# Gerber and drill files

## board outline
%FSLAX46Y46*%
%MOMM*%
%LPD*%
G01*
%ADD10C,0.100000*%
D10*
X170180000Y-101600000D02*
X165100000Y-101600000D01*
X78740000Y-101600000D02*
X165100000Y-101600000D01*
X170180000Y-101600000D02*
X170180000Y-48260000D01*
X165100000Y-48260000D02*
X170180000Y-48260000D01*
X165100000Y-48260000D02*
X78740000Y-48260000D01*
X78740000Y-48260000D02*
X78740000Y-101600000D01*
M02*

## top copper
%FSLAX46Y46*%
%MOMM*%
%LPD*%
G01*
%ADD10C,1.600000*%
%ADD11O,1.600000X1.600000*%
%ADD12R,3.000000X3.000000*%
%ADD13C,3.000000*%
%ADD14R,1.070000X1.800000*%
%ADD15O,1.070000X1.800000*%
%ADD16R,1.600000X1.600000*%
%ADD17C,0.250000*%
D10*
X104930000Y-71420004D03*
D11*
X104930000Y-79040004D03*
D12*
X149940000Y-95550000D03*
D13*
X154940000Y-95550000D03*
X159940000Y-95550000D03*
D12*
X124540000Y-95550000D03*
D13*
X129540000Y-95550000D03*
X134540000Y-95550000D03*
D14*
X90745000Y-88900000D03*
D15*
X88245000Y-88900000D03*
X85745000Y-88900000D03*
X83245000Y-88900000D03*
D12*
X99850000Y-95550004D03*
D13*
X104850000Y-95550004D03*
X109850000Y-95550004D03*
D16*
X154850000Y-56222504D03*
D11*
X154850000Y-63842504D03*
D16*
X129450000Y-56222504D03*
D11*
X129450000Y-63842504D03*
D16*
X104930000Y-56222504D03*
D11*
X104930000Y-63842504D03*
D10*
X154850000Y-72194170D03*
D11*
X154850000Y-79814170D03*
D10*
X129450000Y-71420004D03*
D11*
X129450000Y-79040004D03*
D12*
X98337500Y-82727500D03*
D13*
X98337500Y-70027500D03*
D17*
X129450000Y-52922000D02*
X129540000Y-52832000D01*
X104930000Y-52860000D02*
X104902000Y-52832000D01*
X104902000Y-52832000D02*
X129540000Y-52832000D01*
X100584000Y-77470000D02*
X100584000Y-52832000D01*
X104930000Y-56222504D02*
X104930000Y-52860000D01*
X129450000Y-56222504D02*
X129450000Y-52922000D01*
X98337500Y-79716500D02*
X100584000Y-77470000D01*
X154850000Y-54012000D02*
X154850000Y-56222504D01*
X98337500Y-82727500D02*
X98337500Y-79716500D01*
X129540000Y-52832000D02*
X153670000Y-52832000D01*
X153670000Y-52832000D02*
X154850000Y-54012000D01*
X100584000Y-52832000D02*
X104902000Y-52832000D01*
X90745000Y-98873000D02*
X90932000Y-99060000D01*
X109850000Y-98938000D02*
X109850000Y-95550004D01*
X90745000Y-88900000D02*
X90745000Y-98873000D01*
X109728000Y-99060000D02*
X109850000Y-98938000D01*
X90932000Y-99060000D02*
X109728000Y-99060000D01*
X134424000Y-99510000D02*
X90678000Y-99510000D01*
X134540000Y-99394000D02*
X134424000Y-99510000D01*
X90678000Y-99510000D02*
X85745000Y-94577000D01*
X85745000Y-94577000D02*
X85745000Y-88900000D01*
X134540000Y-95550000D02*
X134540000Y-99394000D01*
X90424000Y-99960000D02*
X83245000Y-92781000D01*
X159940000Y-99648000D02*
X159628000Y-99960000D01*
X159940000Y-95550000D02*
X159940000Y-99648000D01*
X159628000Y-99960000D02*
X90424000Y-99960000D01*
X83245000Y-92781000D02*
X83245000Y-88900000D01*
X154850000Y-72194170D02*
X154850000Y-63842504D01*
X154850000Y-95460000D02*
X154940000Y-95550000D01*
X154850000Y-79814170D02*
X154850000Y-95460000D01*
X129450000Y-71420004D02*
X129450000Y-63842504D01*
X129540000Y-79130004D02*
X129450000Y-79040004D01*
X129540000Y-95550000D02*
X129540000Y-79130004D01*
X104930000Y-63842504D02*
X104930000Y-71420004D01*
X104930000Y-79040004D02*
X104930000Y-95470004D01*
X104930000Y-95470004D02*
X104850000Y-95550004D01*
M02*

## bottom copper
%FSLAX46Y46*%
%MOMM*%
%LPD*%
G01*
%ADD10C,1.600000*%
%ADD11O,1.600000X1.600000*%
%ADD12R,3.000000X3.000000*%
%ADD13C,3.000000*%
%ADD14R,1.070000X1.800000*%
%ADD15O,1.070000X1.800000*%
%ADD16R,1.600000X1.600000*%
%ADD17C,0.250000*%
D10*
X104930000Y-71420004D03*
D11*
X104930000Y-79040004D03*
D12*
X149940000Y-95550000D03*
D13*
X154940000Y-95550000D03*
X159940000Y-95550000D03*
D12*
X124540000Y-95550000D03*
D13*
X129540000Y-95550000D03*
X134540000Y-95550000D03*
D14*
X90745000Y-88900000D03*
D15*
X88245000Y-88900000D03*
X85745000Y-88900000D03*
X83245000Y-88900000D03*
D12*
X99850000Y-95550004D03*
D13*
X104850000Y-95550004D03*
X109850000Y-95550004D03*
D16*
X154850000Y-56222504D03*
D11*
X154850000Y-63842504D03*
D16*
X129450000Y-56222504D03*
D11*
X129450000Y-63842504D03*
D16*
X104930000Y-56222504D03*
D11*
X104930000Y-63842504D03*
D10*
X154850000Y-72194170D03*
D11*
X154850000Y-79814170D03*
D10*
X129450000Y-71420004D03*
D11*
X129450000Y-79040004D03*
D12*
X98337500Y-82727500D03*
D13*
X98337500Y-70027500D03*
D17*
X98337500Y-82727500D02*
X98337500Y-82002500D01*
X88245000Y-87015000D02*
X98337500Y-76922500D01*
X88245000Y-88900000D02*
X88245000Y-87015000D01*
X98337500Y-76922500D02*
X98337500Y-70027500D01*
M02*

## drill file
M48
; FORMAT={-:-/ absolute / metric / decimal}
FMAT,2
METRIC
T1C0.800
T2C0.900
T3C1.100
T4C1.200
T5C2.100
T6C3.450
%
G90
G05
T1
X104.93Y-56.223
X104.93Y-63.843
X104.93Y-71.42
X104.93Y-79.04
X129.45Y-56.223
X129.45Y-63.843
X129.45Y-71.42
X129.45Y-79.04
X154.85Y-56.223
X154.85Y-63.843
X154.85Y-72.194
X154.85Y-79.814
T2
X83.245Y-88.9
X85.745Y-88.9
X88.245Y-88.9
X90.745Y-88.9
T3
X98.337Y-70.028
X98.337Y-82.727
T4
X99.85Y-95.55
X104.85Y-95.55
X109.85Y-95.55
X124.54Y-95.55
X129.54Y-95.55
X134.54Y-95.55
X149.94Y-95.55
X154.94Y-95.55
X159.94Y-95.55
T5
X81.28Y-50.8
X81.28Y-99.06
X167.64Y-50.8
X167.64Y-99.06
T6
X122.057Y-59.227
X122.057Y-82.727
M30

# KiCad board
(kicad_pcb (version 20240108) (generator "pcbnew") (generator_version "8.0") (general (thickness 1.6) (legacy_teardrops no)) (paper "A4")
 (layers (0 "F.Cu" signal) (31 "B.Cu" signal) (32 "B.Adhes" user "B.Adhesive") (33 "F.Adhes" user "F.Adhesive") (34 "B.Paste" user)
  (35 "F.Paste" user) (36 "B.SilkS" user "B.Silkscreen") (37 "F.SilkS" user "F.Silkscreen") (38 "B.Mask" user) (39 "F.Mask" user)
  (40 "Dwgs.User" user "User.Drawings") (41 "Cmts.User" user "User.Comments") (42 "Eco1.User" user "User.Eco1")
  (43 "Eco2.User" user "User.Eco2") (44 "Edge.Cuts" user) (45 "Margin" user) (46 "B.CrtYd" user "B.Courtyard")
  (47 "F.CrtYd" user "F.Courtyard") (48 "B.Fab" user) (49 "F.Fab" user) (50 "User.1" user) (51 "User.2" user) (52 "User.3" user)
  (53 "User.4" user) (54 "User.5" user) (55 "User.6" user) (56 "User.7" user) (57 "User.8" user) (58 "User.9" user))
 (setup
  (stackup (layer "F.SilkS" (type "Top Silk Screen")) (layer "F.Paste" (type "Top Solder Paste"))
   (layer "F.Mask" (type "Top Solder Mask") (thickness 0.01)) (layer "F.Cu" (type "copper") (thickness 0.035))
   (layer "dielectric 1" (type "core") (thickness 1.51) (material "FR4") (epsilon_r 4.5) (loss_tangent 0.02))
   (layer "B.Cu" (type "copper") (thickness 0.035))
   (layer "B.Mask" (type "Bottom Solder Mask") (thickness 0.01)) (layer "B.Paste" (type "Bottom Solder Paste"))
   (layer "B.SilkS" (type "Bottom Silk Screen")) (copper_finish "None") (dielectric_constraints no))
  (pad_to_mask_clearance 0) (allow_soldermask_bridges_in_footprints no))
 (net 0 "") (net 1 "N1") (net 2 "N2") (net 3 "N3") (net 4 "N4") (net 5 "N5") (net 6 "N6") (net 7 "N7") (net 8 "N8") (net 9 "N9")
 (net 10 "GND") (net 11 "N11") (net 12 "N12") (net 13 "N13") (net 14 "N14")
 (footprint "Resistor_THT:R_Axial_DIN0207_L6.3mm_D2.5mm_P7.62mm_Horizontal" (layer "F.Cu") (at 104.93 71.420004 -90)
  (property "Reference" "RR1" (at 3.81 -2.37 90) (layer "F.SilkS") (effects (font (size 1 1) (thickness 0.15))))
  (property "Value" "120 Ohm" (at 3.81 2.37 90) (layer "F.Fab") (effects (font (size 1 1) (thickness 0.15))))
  (pad "1" thru_hole circle (at 0 0 270) (size 1.6 1.6) (drill 0.8) (layers "*.Cu" "*.Mask") (remove_unused_layers no) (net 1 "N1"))
  (pad "2" thru_hole oval (at 7.62 0 270) (size 1.6 1.6) (drill 0.8) (layers "*.Cu" "*.Mask") (remove_unused_layers no) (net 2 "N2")))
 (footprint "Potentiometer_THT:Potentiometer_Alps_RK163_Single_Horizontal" (layer "F.Cu") (at 149.94 95.55 90)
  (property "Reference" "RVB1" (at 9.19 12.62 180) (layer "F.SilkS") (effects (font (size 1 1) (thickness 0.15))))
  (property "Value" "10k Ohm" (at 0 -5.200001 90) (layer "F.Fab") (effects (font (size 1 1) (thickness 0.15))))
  (pad "1" thru_hole rect (at 0 0 270) (size 3 3) (drill 1.2) (layers "*.Cu" "*.Mask") (remove_unused_layers no) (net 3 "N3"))
  (pad "2" thru_hole circle (at 0 5 270) (size 3 3) (drill 1.2) (layers "*.Cu" "*.Mask") (remove_unused_layers no) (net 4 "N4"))
  (pad "3" thru_hole circle (at 0 10 270) (size 3 3) (drill 1.2) (layers "*.Cu" "*.Mask") (remove_unused_layers no) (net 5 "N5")))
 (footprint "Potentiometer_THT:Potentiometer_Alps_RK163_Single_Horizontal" (layer "F.Cu") (at 124.54 95.55 90)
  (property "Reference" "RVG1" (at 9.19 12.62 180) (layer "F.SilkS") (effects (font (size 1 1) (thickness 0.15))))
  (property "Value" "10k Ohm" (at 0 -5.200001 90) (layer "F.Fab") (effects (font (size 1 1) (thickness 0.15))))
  (pad "1" thru_hole rect (at 0 0 270) (size 3 3) (drill 1.2) (layers "*.Cu" "*.Mask") (remove_unused_layers no) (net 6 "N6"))
  (pad "2" thru_hole circle (at 0 5 270) (size 3 3) (drill 1.2) (layers "*.Cu" "*.Mask") (remove_unused_layers no) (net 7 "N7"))
  (pad "3" thru_hole circle (at 0 10 270) (size 3 3) (drill 1.2) (layers "*.Cu" "*.Mask") (remove_unused_layers no) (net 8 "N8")))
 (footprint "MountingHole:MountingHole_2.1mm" (layer "F.Cu") (at 167.64 50.8)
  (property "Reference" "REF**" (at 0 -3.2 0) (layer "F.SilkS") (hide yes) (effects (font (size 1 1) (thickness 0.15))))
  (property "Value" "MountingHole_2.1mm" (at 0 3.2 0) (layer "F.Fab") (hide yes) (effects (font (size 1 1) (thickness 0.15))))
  (pad "" np_thru_hole circle (at 0 0) (size 2.1 2.1) (drill 2.1) (layers "*.Cu" "*.Mask")))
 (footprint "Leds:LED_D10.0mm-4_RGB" (layer "F.Cu") (at 88.9 88.9 180)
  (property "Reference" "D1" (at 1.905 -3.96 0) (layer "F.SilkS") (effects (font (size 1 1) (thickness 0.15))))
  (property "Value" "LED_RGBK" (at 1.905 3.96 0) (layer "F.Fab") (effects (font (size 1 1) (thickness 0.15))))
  (pad "1" thru_hole rect (at -1.845 0 180) (size 1.07 1.8) (drill 0.9) (layers "*.Cu" "*.Mask") (remove_unused_layers no) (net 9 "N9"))
  (pad "2" thru_hole oval (at 0.655 0 180) (size 1.07 1.8) (drill 0.9) (layers "*.Cu" "*.Mask") (remove_unused_layers no) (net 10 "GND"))
  (pad "3" thru_hole oval (at 3.155 0 180) (size 1.07 1.8) (drill 0.9) (layers "*.Cu" "*.Mask") (remove_unused_layers no) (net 8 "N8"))
  (pad "4" thru_hole oval (at 5.655 0 180) (size 1.07 1.8) (drill 0.9) (layers "*.Cu" "*.Mask") (remove_unused_layers no) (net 5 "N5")))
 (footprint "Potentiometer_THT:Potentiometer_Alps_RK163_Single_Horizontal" (layer "F.Cu") (at 99.85 95.550004 90)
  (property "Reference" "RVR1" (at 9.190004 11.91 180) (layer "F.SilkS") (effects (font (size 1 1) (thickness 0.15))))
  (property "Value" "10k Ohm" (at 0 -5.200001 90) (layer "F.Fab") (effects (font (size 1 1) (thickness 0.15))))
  (pad "1" thru_hole rect (at 0 0 270) (size 3 3) (drill 1.2) (layers "*.Cu" "*.Mask") (remove_unused_layers no) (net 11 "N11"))
  (pad "2" thru_hole circle (at 0 5 270) (size 3 3) (drill 1.2) (layers "*.Cu" "*.Mask") (remove_unused_layers no) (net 2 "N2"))
  (pad "3" thru_hole circle (at 0 10 270) (size 3 3) (drill 1.2) (layers "*.Cu" "*.Mask") (remove_unused_layers no) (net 9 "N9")))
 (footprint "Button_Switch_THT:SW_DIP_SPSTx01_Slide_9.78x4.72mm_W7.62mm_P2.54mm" (layer "F.Cu") (at 154.85 56.222504 -90)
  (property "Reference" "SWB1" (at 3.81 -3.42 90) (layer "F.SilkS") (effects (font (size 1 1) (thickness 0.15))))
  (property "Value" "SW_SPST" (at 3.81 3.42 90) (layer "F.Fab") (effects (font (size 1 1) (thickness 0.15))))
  (pad "1" thru_hole rect (at 0 0 270) (size 1.6 1.6) (drill 0.8) (layers "*.Cu" "*.Mask") (remove_unused_layers no) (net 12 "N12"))
  (pad "2" thru_hole oval (at 7.62 0 270) (size 1.6 1.6) (drill 0.8) (layers "*.Cu" "*.Mask") (remove_unused_layers no) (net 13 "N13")))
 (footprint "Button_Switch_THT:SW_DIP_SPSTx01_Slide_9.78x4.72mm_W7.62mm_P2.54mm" (layer "F.Cu") (at 129.45 56.222504 -90)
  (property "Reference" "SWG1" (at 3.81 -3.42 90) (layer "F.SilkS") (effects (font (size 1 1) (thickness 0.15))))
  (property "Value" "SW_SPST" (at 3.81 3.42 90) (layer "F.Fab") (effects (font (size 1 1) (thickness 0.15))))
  (pad "1" thru_hole rect (at 0 0 270) (size 1.6 1.6) (drill 0.8) (layers "*.Cu" "*.Mask") (remove_unused_layers no) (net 12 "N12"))
  (pad "2" thru_hole oval (at 7.62 0 270) (size 1.6 1.6) (drill 0.8) (layers "*.Cu" "*.Mask") (remove_unused_layers no) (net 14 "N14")))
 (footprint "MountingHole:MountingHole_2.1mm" (layer "F.Cu") (at 81.28 50.8)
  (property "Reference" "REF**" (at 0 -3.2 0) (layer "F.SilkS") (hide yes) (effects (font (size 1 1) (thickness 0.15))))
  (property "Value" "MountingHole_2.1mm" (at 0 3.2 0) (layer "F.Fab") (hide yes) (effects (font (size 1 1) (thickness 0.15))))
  (pad "" np_thru_hole circle (at 0 0) (size 2.1 2.1) (drill 2.1) (layers "*.Cu" "*.Mask")))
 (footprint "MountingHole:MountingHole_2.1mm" (layer "F.Cu") (at 81.28 99.06)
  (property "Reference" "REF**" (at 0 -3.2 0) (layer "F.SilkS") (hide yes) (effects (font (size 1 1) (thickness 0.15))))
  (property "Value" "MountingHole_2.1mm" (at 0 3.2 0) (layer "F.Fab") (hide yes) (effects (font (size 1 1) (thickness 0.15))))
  (pad "" np_thru_hole circle (at 0 0) (size 2.1 2.1) (drill 2.1) (layers "*.Cu" "*.Mask")))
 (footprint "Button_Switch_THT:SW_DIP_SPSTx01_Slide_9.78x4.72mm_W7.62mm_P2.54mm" (layer "F.Cu") (at 104.93 56.222504 -90)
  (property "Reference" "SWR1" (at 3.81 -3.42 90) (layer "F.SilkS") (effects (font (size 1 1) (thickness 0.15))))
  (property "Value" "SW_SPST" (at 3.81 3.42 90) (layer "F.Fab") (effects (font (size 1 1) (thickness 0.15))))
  (pad "1" thru_hole rect (at 0 0 270) (size 1.6 1.6) (drill 0.8) (layers "*.Cu" "*.Mask") (remove_unused_layers no) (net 12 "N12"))
  (pad "2" thru_hole oval (at 7.62 0 270) (size 1.6 1.6) (drill 0.8) (layers "*.Cu" "*.Mask") (remove_unused_layers no) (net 1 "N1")))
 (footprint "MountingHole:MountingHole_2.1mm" (layer "F.Cu") (at 167.64 99.06)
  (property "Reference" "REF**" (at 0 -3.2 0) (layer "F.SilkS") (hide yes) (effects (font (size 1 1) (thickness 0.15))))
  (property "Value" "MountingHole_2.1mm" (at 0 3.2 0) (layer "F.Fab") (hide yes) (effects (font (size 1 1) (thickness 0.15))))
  (pad "" np_thru_hole circle (at 0 0) (size 2.1 2.1) (drill 2.1) (layers "*.Cu" "*.Mask")))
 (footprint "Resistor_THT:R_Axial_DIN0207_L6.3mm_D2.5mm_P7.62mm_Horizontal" (layer "F.Cu") (at 154.85 72.19417 -90)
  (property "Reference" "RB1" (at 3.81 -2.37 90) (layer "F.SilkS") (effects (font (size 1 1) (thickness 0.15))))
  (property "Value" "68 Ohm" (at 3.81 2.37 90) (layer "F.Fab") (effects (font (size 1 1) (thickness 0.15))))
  (pad "1" thru_hole circle (at 0 0 270) (size 1.6 1.6) (drill 0.8) (layers "*.Cu" "*.Mask") (remove_unused_layers no) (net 13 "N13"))
  (pad "2" thru_hole oval (at 7.62 0 270) (size 1.6 1.6) (drill 0.8) (layers "*.Cu" "*.Mask") (remove_unused_layers no) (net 4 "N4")))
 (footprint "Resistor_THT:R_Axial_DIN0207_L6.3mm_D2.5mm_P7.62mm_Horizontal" (layer "F.Cu") (at 129.45 71.420004 -90)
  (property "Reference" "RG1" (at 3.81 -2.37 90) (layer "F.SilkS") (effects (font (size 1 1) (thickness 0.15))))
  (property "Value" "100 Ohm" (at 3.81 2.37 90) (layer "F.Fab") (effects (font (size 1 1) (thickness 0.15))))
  (pad "1" thru_hole circle (at 0 0 270) (size 1.6 1.6) (drill 0.8) (layers "*.Cu" "*.Mask") (remove_unused_layers no) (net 14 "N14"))
  (pad "2" thru_hole oval (at 7.62 0 270) (size 1.6 1.6) (drill 0.8) (layers "*.Cu" "*.Mask") (remove_unused_layers no) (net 7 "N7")))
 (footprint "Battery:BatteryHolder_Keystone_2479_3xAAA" (layer "B.Cu") (at 98.3375 82.7275)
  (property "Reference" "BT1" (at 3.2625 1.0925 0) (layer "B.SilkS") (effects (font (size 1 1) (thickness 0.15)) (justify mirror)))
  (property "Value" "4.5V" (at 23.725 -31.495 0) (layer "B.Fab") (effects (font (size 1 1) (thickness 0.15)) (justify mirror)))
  (pad "" np_thru_hole circle (at 23.72 -23.5) (size 3.45 3.45) (drill 3.45) (layers "*.Cu" "*.Mask"))
  (pad "" np_thru_hole circle (at 23.72 0) (size 3.45 3.45) (drill 3.45) (layers "*.Cu" "*.Mask"))
  (pad "1" thru_hole rect (at 0 0) (size 3 3) (drill 1.1) (layers "*.Cu" "*.Mask") (remove_unused_layers no) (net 12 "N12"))
  (pad "2" thru_hole circle (at 0 -12.7) (size 3 3) (drill 1.1) (layers "*.Cu" "*.Mask") (remove_unused_layers no) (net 10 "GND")))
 (gr_line (start 170.18 101.6) (end 165.1 101.6) (stroke (width 0.1) (type solid)) (layer "Edge.Cuts"))
 (gr_line (start 78.74 101.6) (end 165.1 101.6) (stroke (width 0.1) (type solid)) (layer "Edge.Cuts"))
 (gr_line (start 170.18 101.6) (end 170.18 48.26) (stroke (width 0.1) (type solid)) (layer "Edge.Cuts"))
 (gr_line (start 165.1 48.26) (end 170.18 48.26) (stroke (width 0.1) (type solid)) (layer "Edge.Cuts"))
 (gr_line (start 165.1 48.26) (end 78.74 48.26) (stroke (width 0.1) (type solid)) (layer "Edge.Cuts"))
 (gr_line (start 78.74 48.26) (end 78.74 101.6) (stroke (width 0.1) (type solid)) (layer "Edge.Cuts"))
 (segment (start 129.45 52.922) (end 129.54 52.832) (width 0.25) (layer "F.Cu") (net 12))
 (segment (start 104.93 52.86) (end 104.902 52.832) (width 0.25) (layer "F.Cu") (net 12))
 (segment (start 104.902 52.832) (end 129.54 52.832) (width 0.25) (layer "F.Cu") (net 12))
 (segment (start 100.584 77.47) (end 100.584 52.832) (width 0.25) (layer "F.Cu") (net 12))
 (segment (start 104.93 56.222504) (end 104.93 52.86) (width 0.25) (layer "F.Cu") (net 12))
 (segment (start 129.45 56.222504) (end 129.45 52.922) (width 0.25) (layer "F.Cu") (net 12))
 (segment (start 98.3375 79.7165) (end 100.584 77.47) (width 0.25) (layer "F.Cu") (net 12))
 (segment (start 154.85 54.012) (end 154.85 56.222504) (width 0.25) (layer "F.Cu") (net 12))
 (segment (start 98.3375 82.7275) (end 98.3375 79.7165) (width 0.25) (layer "F.Cu") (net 12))
 (segment (start 129.54 52.832) (end 153.67 52.832) (width 0.25) (layer "F.Cu") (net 12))
 (segment (start 153.67 52.832) (end 154.85 54.012) (width 0.25) (layer "F.Cu") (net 12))
 (segment (start 100.584 52.832) (end 104.902 52.832) (width 0.25) (layer "F.Cu") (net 12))
 (segment (start 98.3375 82.7275) (end 98.3375 82.0025) (width 0.25) (layer "B.Cu") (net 12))
 (segment (start 88.245 87.015) (end 98.3375 76.9225) (width 0.25) (layer "B.Cu") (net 10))
 (segment (start 88.245 88.9) (end 88.245 87.015) (width 0.25) (layer "B.Cu") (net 10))
 (segment (start 98.3375 76.9225) (end 98.3375 70.0275) (width 0.25) (layer "B.Cu") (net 10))
 (segment (start 90.745 98.873) (end 90.932 99.06) (width 0.25) (layer "F.Cu") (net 9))
 (segment (start 109.85 98.938) (end 109.85 95.550004) (width 0.25) (layer "F.Cu") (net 9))
 (segment (start 90.745 88.9) (end 90.745 98.873) (width 0.25) (layer "F.Cu") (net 9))
 (segment (start 109.728 99.06) (end 109.85 98.938) (width 0.25) (layer "F.Cu") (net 9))
 (segment (start 90.932 99.06) (end 109.728 99.06) (width 0.25) (layer "F.Cu") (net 9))
 (segment (start 134.424 99.51) (end 90.678 99.51) (width 0.25) (layer "F.Cu") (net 8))
 (segment (start 134.54 99.394) (end 134.424 99.51) (width 0.25) (layer "F.Cu") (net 8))
 (segment (start 90.678 99.51) (end 85.745 94.577) (width 0.25) (layer "F.Cu") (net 8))
 (segment (start 85.745 94.577) (end 85.745 88.9) (width 0.25) (layer "F.Cu") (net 8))
 (segment (start 134.54 95.55) (end 134.54 99.394) (width 0.25) (layer "F.Cu") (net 8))
 (segment (start 90.424 99.96) (end 83.245 92.781) (width 0.25) (layer "F.Cu") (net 5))
 (segment (start 159.94 99.648) (end 159.628 99.96) (width 0.25) (layer "F.Cu") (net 5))
 (segment (start 159.94 95.55) (end 159.94 99.648) (width 0.25) (layer "F.Cu") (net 5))
 (segment (start 159.628 99.96) (end 90.424 99.96) (width 0.25) (layer "F.Cu") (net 5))
 (segment (start 83.245 92.781) (end 83.245 88.9) (width 0.25) (layer "F.Cu") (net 5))
 (segment (start 154.85 72.19417) (end 154.85 63.842504) (width 0.25) (layer "F.Cu") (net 13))
 (segment (start 154.85 95.46) (end 154.94 95.55) (width 0.25) (layer "F.Cu") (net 4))
 (segment (start 154.85 79.81417) (end 154.85 95.46) (width 0.25) (layer "F.Cu") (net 4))
 (segment (start 129.45 71.420004) (end 129.45 63.842504) (width 0.25) (layer "F.Cu") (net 14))
 (segment (start 129.54 79.130004) (end 129.45 79.040004) (width 0.25) (layer "F.Cu") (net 7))
 (segment (start 129.54 95.55) (end 129.54 79.130004) (width 0.25) (layer "F.Cu") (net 7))
 (segment (start 104.93 63.842504) (end 104.93 71.420004) (width 0.25) (layer "F.Cu") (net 1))
 (segment (start 104.93 79.040004) (end 104.93 95.470004) (width 0.25) (layer "F.Cu") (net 2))
 (segment (start 104.93 95.470004) (end 104.85 95.550004) (width 0.25) (layer "F.Cu") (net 2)))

